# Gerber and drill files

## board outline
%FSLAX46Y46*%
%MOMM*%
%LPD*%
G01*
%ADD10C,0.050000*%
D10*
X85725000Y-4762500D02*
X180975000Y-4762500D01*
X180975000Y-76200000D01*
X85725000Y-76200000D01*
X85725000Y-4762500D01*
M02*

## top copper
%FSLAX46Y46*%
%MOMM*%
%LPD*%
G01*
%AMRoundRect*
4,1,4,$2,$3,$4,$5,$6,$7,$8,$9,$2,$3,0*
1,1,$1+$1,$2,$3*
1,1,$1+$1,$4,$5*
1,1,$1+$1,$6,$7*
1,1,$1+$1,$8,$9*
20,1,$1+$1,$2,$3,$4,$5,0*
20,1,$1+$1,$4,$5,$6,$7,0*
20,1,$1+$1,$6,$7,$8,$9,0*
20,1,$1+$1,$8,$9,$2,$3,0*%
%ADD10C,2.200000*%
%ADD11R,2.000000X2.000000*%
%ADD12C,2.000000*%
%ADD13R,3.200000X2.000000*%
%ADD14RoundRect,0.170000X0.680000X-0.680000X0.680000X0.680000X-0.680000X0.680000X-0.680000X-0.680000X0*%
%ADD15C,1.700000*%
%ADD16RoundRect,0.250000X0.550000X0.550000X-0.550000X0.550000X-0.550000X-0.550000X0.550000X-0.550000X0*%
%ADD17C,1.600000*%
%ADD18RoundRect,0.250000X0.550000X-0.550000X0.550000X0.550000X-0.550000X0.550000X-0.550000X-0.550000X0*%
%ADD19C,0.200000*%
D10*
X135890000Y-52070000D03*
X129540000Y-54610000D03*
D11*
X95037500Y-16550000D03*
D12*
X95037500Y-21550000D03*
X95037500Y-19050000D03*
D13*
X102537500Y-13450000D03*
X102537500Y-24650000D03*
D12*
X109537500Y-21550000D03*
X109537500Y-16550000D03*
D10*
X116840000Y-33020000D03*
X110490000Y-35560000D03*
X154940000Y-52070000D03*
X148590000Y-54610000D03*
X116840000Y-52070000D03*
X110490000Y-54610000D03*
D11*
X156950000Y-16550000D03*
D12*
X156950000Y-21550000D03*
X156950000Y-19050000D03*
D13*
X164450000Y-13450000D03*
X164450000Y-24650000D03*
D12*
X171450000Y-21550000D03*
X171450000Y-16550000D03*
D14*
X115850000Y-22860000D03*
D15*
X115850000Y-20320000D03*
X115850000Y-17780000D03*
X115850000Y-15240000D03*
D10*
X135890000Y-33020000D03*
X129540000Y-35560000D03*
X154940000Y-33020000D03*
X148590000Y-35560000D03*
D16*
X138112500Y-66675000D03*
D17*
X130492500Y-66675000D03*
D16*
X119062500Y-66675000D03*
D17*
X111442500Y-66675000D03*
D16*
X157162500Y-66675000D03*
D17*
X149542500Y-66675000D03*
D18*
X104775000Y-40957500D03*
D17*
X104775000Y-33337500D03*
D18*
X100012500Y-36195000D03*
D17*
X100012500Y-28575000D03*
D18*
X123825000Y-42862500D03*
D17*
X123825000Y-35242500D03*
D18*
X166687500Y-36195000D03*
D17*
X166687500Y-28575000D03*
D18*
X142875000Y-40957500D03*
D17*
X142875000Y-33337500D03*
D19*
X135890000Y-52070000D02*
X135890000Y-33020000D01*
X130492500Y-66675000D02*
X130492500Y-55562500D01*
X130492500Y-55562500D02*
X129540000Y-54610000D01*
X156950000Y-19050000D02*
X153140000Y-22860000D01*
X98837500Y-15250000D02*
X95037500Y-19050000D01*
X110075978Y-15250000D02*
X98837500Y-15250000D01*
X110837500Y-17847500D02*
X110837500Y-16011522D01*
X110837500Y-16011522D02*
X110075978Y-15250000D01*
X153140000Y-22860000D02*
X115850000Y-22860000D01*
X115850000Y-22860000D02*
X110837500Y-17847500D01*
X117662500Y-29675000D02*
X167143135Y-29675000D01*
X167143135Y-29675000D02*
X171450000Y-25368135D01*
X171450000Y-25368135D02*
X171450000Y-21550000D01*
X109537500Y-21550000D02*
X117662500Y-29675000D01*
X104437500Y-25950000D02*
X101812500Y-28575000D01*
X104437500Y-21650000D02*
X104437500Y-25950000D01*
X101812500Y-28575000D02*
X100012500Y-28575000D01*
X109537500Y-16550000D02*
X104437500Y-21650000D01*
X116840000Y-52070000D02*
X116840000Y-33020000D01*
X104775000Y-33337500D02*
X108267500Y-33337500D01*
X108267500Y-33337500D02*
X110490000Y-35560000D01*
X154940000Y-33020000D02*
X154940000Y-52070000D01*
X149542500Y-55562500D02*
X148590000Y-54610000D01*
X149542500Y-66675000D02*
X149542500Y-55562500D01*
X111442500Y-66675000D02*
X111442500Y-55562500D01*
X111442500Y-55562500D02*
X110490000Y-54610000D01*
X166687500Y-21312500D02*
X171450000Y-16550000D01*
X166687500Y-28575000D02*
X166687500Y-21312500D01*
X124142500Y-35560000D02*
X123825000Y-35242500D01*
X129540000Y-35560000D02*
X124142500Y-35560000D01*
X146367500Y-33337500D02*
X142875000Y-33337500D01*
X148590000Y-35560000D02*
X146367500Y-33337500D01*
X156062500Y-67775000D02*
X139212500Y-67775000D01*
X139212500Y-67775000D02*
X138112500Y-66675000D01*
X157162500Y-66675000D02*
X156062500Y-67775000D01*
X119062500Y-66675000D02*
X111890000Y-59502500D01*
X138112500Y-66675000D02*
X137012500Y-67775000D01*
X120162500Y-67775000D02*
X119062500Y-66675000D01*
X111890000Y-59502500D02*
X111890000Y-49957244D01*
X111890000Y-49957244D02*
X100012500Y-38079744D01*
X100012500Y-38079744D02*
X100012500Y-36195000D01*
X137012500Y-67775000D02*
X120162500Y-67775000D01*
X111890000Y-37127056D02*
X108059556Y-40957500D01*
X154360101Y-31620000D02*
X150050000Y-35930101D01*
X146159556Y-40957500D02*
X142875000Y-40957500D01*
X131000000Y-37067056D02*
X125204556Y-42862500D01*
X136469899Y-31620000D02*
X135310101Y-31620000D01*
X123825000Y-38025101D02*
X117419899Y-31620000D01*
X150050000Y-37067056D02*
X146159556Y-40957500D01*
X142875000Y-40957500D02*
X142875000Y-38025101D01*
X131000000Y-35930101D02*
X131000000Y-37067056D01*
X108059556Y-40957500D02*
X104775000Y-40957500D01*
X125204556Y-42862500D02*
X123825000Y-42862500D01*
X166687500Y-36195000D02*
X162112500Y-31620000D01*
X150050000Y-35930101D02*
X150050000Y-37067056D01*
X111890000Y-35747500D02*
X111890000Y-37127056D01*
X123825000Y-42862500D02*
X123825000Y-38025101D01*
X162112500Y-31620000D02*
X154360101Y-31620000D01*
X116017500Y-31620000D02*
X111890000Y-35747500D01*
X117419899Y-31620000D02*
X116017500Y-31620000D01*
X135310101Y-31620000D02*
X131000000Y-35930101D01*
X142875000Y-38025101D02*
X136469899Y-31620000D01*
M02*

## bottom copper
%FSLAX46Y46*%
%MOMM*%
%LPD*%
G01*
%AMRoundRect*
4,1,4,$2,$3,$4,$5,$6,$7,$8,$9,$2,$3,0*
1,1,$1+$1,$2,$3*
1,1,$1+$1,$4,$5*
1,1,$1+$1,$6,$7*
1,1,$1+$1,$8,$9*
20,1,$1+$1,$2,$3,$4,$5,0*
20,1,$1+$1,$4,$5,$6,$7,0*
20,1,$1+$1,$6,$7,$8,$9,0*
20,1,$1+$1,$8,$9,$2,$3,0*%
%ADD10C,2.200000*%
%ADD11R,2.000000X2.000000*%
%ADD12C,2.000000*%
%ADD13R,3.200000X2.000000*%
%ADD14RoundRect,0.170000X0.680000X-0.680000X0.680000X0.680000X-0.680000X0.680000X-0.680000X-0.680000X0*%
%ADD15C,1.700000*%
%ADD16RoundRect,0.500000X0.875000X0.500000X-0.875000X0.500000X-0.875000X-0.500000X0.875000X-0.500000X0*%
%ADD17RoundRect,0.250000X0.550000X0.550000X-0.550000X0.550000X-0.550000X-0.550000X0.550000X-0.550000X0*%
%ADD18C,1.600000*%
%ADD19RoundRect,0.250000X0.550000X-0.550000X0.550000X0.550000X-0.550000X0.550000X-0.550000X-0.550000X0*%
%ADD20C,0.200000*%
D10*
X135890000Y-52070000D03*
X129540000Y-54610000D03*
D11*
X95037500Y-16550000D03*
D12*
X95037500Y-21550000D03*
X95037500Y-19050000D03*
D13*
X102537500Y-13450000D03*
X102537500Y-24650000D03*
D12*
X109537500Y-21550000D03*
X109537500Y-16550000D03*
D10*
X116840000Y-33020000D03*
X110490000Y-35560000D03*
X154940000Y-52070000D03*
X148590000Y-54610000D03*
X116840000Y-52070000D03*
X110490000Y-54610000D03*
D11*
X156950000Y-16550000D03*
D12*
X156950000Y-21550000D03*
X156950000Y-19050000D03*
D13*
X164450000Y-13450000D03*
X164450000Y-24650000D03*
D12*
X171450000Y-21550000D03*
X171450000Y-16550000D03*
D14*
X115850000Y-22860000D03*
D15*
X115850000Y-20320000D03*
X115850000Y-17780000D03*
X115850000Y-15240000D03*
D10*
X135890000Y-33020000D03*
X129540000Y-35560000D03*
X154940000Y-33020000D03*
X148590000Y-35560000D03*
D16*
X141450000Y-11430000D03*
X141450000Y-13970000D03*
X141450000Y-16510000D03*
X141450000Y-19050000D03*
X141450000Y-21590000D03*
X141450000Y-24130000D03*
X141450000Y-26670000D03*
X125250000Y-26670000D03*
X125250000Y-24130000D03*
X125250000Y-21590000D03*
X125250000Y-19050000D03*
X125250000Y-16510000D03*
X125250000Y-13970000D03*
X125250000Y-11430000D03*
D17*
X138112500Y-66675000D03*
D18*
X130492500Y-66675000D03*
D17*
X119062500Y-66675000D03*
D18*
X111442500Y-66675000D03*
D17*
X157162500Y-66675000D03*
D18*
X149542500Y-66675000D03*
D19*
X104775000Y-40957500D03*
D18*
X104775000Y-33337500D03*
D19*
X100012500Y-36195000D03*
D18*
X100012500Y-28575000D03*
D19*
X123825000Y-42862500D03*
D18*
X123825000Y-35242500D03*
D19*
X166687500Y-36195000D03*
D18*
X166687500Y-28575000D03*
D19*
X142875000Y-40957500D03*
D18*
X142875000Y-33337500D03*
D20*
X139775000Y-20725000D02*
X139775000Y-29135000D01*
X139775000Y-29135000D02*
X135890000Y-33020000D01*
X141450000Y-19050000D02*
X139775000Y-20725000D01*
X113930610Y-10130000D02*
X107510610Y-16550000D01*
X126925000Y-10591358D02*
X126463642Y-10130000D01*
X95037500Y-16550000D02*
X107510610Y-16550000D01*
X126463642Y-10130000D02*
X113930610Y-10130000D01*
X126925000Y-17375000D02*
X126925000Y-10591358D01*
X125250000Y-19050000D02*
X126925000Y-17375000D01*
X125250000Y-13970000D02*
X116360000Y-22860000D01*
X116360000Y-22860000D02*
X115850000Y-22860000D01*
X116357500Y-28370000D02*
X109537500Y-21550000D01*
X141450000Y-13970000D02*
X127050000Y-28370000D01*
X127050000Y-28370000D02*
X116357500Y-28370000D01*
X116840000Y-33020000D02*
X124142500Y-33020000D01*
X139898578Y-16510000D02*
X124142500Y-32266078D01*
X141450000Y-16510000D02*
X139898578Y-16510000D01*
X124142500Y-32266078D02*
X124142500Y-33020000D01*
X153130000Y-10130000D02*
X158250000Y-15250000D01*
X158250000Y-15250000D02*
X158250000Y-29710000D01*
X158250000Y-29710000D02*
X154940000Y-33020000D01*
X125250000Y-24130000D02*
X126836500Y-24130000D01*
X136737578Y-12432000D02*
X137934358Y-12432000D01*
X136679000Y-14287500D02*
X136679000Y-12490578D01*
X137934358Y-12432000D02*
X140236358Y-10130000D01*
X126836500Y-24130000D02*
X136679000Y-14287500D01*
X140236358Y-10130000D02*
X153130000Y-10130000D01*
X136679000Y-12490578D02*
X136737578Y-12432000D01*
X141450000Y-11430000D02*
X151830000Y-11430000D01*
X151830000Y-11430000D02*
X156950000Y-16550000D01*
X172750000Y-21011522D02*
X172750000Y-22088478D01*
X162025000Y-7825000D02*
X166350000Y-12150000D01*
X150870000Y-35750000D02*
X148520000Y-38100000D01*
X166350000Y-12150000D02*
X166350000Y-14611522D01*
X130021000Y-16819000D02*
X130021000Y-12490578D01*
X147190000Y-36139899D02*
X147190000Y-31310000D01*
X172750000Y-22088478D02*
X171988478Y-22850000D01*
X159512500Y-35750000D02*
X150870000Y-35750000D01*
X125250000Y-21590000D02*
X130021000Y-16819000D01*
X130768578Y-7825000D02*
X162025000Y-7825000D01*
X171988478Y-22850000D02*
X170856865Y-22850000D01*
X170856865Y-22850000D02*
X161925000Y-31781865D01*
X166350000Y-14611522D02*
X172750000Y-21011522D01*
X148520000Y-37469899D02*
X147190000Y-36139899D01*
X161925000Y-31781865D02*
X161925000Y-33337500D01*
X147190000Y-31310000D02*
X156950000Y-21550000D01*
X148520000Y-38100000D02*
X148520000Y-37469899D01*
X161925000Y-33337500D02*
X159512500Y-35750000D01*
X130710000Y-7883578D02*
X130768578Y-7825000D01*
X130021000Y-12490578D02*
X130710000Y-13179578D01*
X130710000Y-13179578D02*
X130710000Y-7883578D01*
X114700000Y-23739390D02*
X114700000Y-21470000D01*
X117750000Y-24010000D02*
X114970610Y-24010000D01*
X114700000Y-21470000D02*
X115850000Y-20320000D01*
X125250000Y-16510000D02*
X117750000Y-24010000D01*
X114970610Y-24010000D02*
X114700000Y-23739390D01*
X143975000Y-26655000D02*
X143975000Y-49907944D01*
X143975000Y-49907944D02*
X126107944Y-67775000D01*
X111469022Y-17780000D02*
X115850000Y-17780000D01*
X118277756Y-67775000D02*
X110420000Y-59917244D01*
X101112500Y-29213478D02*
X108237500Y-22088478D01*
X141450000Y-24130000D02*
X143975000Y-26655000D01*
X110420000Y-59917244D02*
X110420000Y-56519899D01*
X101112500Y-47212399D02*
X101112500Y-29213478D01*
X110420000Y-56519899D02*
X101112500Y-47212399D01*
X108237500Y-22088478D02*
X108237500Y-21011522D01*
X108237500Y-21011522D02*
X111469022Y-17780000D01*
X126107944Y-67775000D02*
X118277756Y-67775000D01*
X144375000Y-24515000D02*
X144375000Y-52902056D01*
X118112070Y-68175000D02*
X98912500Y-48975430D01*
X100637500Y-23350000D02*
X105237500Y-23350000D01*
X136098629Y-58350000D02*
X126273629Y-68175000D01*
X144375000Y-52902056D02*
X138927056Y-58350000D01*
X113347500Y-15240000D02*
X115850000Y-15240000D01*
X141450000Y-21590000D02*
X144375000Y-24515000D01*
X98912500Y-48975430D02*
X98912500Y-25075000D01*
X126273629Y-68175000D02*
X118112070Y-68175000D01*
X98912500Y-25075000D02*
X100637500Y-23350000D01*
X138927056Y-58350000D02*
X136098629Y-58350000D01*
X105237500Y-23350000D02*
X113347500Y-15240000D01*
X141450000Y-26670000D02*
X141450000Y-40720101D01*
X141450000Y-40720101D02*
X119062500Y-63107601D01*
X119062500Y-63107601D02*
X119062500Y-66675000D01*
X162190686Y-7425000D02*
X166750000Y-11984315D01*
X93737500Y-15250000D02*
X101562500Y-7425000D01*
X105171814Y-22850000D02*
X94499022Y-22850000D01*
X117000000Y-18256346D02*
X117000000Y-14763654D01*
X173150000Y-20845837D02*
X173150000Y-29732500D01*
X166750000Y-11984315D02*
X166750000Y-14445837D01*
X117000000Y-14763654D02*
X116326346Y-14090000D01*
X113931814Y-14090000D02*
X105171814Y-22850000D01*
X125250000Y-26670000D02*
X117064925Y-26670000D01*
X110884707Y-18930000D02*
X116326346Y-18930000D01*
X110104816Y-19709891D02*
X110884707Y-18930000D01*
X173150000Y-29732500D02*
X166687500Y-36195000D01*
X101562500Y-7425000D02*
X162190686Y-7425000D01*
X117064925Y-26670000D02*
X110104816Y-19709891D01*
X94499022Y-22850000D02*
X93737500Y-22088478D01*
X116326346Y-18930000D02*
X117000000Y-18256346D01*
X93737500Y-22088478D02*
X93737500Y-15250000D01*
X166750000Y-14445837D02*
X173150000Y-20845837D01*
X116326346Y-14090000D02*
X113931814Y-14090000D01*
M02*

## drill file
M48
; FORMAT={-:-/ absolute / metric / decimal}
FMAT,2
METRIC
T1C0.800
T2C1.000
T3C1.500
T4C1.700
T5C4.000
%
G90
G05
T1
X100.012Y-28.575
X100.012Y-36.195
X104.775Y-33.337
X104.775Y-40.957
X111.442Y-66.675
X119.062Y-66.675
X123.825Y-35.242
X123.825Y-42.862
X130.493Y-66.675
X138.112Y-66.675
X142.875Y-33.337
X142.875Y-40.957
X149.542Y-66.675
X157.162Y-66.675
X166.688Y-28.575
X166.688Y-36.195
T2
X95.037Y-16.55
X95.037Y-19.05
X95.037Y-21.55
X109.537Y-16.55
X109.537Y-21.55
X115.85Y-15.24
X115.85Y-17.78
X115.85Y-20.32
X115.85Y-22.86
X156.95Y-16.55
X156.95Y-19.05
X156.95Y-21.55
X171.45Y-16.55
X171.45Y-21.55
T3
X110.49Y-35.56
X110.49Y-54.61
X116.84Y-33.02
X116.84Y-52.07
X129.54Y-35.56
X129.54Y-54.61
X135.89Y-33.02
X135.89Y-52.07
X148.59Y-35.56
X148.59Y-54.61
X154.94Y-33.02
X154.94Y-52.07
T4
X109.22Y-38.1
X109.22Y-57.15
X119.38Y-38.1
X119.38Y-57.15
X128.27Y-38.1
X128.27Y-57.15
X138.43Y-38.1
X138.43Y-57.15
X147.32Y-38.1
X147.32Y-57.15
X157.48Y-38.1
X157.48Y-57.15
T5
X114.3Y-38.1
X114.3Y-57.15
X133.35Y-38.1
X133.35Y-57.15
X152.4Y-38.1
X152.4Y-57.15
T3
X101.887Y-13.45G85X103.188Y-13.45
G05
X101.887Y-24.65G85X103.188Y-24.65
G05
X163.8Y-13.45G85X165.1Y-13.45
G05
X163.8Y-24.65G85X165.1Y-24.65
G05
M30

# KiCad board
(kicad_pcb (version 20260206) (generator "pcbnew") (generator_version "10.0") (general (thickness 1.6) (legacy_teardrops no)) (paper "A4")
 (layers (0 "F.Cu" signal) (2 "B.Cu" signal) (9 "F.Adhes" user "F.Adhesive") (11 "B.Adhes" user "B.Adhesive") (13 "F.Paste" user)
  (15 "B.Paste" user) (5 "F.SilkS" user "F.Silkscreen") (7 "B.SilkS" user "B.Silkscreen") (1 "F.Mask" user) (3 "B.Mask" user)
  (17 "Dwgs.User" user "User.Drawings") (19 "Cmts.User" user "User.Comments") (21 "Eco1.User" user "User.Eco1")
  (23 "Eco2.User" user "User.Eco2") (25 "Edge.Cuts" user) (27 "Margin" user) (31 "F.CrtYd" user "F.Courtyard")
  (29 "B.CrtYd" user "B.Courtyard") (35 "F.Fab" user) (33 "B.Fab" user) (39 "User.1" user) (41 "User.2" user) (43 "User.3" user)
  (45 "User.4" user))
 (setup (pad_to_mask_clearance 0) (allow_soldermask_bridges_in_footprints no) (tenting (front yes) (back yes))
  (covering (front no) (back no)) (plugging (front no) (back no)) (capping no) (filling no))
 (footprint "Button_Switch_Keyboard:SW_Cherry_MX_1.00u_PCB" (layer "F.Cu") (at 135.89 52.07)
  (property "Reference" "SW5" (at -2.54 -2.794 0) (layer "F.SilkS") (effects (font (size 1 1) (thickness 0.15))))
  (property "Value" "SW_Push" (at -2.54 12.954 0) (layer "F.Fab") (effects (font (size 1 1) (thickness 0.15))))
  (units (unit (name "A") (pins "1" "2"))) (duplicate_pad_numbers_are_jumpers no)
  (pad "" np_thru_hole circle (at -7.62 5.08) (size 1.7 1.7) (drill 1.7) (layers "*.Cu" "*.Mask"))
  (pad "" np_thru_hole circle (at -2.54 5.08) (size 4 4) (drill 4) (layers "*.Cu" "*.Mask"))
  (pad "" np_thru_hole circle (at 2.54 5.08) (size 1.7 1.7) (drill 1.7) (layers "*.Cu" "*.Mask"))
  (pad "1" thru_hole circle (at 0 0) (size 2.2 2.2) (drill 1.5) (layers "*.Cu" "*.Mask") (remove_unused_layers no) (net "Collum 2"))
  (pad "2" thru_hole circle (at -6.35 2.54) (size 2.2 2.2) (drill 1.5) (layers "*.Cu" "*.Mask") (remove_unused_layers no) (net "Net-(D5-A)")))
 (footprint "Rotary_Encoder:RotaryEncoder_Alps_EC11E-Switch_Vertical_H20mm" (layer "F.Cu") (at 95.0375 16.55)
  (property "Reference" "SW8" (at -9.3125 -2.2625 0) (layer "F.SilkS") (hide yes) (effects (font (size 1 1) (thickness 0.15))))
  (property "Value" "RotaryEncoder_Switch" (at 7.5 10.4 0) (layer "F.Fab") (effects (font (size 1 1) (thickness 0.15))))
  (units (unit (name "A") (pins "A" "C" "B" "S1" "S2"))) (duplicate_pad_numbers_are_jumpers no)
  (pad "A" thru_hole rect (at 0 0) (size 2 2) (drill 1) (layers "*.Cu" "*.Mask") (remove_unused_layers no) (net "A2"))
  (pad "B" thru_hole circle (at 0 5) (size 2 2) (drill 1) (layers "*.Cu" "*.Mask") (remove_unused_layers no) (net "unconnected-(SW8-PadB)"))
  (pad "C" thru_hole circle (at 0 2.5) (size 2 2) (drill 1) (layers "*.Cu" "*.Mask") (remove_unused_layers no) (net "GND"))
  (pad "MP" thru_hole rect (at 7.5 -3.1) (size 3.2 2) (drill oval 2.8 1.5) (layers "*.Cu" "*.Mask") (remove_unused_layers no))
  (pad "MP" thru_hole rect (at 7.5 8.1) (size 3.2 2) (drill oval 2.8 1.5) (layers "*.Cu" "*.Mask") (remove_unused_layers no))
  (pad "S1" thru_hole circle (at 14.5 5) (size 2 2) (drill 1) (layers "*.Cu" "*.Mask") (remove_unused_layers no) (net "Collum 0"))
  (pad "S2" thru_hole circle (at 14.5 0) (size 2 2) (drill 1) (layers "*.Cu" "*.Mask") (remove_unused_layers no) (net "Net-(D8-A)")))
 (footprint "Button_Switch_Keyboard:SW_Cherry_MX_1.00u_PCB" (layer "F.Cu") (at 116.84 33.02)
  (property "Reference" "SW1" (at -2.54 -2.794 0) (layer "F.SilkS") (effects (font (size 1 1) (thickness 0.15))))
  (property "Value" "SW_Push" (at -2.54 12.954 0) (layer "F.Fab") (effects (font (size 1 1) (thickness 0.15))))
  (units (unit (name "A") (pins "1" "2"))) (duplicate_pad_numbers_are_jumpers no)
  (pad "" np_thru_hole circle (at -7.62 5.08) (size 1.7 1.7) (drill 1.7) (layers "*.Cu" "*.Mask"))
  (pad "" np_thru_hole circle (at -2.54 5.08) (size 4 4) (drill 4) (layers "*.Cu" "*.Mask"))
  (pad "" np_thru_hole circle (at 2.54 5.08) (size 1.7 1.7) (drill 1.7) (layers "*.Cu" "*.Mask"))
  (pad "1" thru_hole circle (at 0 0) (size 2.2 2.2) (drill 1.5) (layers "*.Cu" "*.Mask") (remove_unused_layers no) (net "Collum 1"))
  (pad "2" thru_hole circle (at -6.35 2.54) (size 2.2 2.2) (drill 1.5) (layers "*.Cu" "*.Mask") (remove_unused_layers no) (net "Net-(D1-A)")))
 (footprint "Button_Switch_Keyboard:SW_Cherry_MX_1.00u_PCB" (layer "F.Cu") (at 154.94 52.07)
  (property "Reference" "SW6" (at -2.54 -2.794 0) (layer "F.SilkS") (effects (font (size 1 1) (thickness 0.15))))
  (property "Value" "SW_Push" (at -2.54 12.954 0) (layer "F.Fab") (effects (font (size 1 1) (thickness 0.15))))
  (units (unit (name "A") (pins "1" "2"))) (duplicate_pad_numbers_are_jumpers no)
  (pad "" np_thru_hole circle (at -7.62 5.08) (size 1.7 1.7) (drill 1.7) (layers "*.Cu" "*.Mask"))
  (pad "" np_thru_hole circle (at -2.54 5.08) (size 4 4) (drill 4) (layers "*.Cu" "*.Mask"))
  (pad "" np_thru_hole circle (at 2.54 5.08) (size 1.7 1.7) (drill 1.7) (layers "*.Cu" "*.Mask"))
  (pad "1" thru_hole circle (at 0 0) (size 2.2 2.2) (drill 1.5) (layers "*.Cu" "*.Mask") (remove_unused_layers no) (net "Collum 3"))
  (pad "2" thru_hole circle (at -6.35 2.54) (size 2.2 2.2) (drill 1.5) (layers "*.Cu" "*.Mask") (remove_unused_layers no) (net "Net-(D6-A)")))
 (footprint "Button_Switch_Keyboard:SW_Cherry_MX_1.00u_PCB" (layer "F.Cu") (at 116.84 52.07)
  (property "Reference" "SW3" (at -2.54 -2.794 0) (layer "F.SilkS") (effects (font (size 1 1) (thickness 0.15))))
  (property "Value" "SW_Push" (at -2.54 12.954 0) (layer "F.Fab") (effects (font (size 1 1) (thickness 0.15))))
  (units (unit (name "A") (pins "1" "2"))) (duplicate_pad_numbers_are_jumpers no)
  (pad "" np_thru_hole circle (at -7.62 5.08) (size 1.7 1.7) (drill 1.7) (layers "*.Cu" "*.Mask"))
  (pad "" np_thru_hole circle (at -2.54 5.08) (size 4 4) (drill 4) (layers "*.Cu" "*.Mask"))
  (pad "" np_thru_hole circle (at 2.54 5.08) (size 1.7 1.7) (drill 1.7) (layers "*.Cu" "*.Mask"))
  (pad "1" thru_hole circle (at 0 0) (size 2.2 2.2) (drill 1.5) (layers "*.Cu" "*.Mask") (remove_unused_layers no) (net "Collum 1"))
  (pad "2" thru_hole circle (at -6.35 2.54) (size 2.2 2.2) (drill 1.5) (layers "*.Cu" "*.Mask") (remove_unused_layers no) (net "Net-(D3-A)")))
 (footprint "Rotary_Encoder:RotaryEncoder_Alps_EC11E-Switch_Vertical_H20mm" (layer "F.Cu") (at 156.95 16.55)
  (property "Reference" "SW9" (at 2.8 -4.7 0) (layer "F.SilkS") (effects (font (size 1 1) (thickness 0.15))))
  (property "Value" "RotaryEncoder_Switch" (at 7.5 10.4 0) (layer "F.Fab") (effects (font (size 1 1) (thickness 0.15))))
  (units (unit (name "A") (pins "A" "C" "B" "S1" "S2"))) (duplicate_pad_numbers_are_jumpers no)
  (pad "A" thru_hole rect (at 0 0) (size 2 2) (drill 1) (layers "*.Cu" "*.Mask") (remove_unused_layers no) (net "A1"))
  (pad "B" thru_hole circle (at 0 5) (size 2 2) (drill 1) (layers "*.Cu" "*.Mask") (remove_unused_layers no) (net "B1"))
  (pad "C" thru_hole circle (at 0 2.5) (size 2 2) (drill 1) (layers "*.Cu" "*.Mask") (remove_unused_layers no) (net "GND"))
  (pad "MP" thru_hole rect (at 7.5 -3.1) (size 3.2 2) (drill oval 2.8 1.5) (layers "*.Cu" "*.Mask") (remove_unused_layers no))
  (pad "MP" thru_hole rect (at 7.5 8.1) (size 3.2 2) (drill oval 2.8 1.5) (layers "*.Cu" "*.Mask") (remove_unused_layers no))
  (pad "S1" thru_hole circle (at 14.5 5) (size 2 2) (drill 1) (layers "*.Cu" "*.Mask") (remove_unused_layers no) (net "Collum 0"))
  (pad "S2" thru_hole circle (at 14.5 0) (size 2 2) (drill 1) (layers "*.Cu" "*.Mask") (remove_unused_layers no) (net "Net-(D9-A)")))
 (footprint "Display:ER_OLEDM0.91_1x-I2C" (layer "F.Cu") (at 115.85 22.86 90)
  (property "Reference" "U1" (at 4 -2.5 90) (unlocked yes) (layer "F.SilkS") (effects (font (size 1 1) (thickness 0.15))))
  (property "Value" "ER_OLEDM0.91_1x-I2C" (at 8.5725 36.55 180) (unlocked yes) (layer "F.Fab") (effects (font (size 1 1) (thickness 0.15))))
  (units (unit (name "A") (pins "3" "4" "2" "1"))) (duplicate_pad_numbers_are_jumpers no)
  (pad "1" thru_hole roundrect (at 0 0 90) (size 1.7 1.7) (drill 1) (layers "*.Cu" "*.Mask") (remove_unused_layers no)
   (roundrect_rratio 0.1) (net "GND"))
  (pad "2" thru_hole circle (at 2.54 0 90) (size 1.7 1.7) (drill 1) (layers "*.Cu" "*.Mask") (remove_unused_layers no) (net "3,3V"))
  (pad "3" thru_hole circle (at 5.08 0 90) (size 1.7 1.7) (drill 1) (layers "*.Cu" "*.Mask") (remove_unused_layers no) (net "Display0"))
  (pad "4" thru_hole circle (at 7.62 0 90) (size 1.7 1.7) (drill 1) (layers "*.Cu" "*.Mask") (remove_unused_layers no) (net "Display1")))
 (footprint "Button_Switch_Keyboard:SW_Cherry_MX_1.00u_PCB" (layer "F.Cu") (at 135.89 33.02)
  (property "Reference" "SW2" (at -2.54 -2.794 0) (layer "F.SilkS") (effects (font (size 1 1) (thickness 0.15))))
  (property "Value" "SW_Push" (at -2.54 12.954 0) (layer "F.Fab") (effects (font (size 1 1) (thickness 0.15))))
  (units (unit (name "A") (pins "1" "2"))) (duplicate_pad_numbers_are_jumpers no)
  (pad "" np_thru_hole circle (at -7.62 5.08) (size 1.7 1.7) (drill 1.7) (layers "*.Cu" "*.Mask"))
  (pad "" np_thru_hole circle (at -2.54 5.08) (size 4 4) (drill 4) (layers "*.Cu" "*.Mask"))
  (pad "" np_thru_hole circle (at 2.54 5.08) (size 1.7 1.7) (drill 1.7) (layers "*.Cu" "*.Mask"))
  (pad "1" thru_hole circle (at 0 0) (size 2.2 2.2) (drill 1.5) (layers "*.Cu" "*.Mask") (remove_unused_layers no) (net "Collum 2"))
  (pad "2" thru_hole circle (at -6.35 2.54) (size 2.2 2.2) (drill 1.5) (layers "*.Cu" "*.Mask") (remove_unused_layers no) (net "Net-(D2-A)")))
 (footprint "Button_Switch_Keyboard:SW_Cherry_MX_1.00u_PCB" (layer "F.Cu") (at 154.94 33.02)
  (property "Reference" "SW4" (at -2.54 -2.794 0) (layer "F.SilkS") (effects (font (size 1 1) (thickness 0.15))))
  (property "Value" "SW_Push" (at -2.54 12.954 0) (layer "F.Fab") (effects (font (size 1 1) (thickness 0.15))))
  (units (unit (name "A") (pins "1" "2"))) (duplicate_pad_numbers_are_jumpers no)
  (pad "" np_thru_hole circle (at -7.62 5.08) (size 1.7 1.7) (drill 1.7) (layers "*.Cu" "*.Mask"))
  (pad "" np_thru_hole circle (at -2.54 5.08) (size 4 4) (drill 4) (layers "*.Cu" "*.Mask"))
  (pad "" np_thru_hole circle (at 2.54 5.08) (size 1.7 1.7) (drill 1.7) (layers "*.Cu" "*.Mask"))
  (pad "1" thru_hole circle (at 0 0) (size 2.2 2.2) (drill 1.5) (layers "*.Cu" "*.Mask") (remove_unused_layers no) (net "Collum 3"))
  (pad "2" thru_hole circle (at -6.35 2.54) (size 2.2 2.2) (drill 1.5) (layers "*.Cu" "*.Mask") (remove_unused_layers no) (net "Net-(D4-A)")))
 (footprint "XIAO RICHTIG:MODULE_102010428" (layer "B.Cu") (at 133.35 19.05 180)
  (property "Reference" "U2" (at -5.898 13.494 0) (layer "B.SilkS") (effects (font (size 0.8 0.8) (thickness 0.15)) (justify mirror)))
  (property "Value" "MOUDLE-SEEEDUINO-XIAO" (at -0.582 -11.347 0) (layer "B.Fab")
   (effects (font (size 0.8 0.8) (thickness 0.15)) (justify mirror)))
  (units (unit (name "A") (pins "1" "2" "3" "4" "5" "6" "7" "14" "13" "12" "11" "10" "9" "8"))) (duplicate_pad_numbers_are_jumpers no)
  (pad "1" smd roundrect (at -8.1 7.62 180) (size 2.75 2) (layers "B.Cu" "B.Mask" "B.Paste") (roundrect_rratio 0.25) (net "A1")
   (solder_mask_margin 0.102))
  (pad "2" smd roundrect (at -8.1 5.08 180) (size 2.75 2) (layers "B.Cu" "B.Mask" "B.Paste") (roundrect_rratio 0.25) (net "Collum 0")
   (solder_mask_margin 0.102))
  (pad "3" smd roundrect (at -8.1 2.54 180) (size 2.75 2) (layers "B.Cu" "B.Mask" "B.Paste") (roundrect_rratio 0.25) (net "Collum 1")
   (solder_mask_margin 0.102))
  (pad "4" smd roundrect (at -8.1 0 180) (size 2.75 2) (layers "B.Cu" "B.Mask" "B.Paste") (roundrect_rratio 0.25) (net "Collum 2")
   (solder_mask_margin 0.102))
  (pad "5" smd roundrect (at -8.1 -2.54 180) (size 2.75 2) (layers "B.Cu" "B.Mask" "B.Paste") (roundrect_rratio 0.25) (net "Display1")
   (solder_mask_margin 0.102))
  (pad "6" smd roundrect (at -8.1 -5.08 180) (size 2.75 2) (layers "B.Cu" "B.Mask" "B.Paste") (roundrect_rratio 0.25) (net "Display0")
   (solder_mask_margin 0.102))
  (pad "7" smd roundrect (at -8.1 -7.62 180) (size 2.75 2) (layers "B.Cu" "B.Mask" "B.Paste") (roundrect_rratio 0.25) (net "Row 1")
   (solder_mask_margin 0.102))
  (pad "8" smd roundrect (at 8.1 -7.62 180) (size 2.75 2) (layers "B.Cu" "B.Mask" "B.Paste") (roundrect_rratio 0.25) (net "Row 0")
   (solder_mask_margin 0.102))
  (pad "9" smd roundrect (at 8.1 -5.08 180) (size 2.75 2) (layers "B.Cu" "B.Mask" "B.Paste") (roundrect_rratio 0.25) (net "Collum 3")
   (solder_mask_margin 0.102))
  (pad "10" smd roundrect (at 8.1 -2.54 180) (size 2.75 2) (layers "B.Cu" "B.Mask" "B.Paste") (roundrect_rratio 0.25) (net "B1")
   (solder_mask_margin 0.102))
  (pad "11" smd roundrect (at 8.1 0 180) (size 2.75 2) (layers "B.Cu" "B.Mask" "B.Paste") (roundrect_rratio 0.25) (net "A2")
   (solder_mask_margin 0.102))
  (pad "12" smd roundrect (at 8.1 2.54 180) (size 2.75 2) (layers "B.Cu" "B.Mask" "B.Paste") (roundrect_rratio 0.25) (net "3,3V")
   (solder_mask_margin 0.102))
  (pad "13" smd roundrect (at 8.1 5.08 180) (size 2.75 2) (layers "B.Cu" "B.Mask" "B.Paste") (roundrect_rratio 0.25) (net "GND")
   (solder_mask_margin 0.102))
  (pad "14" smd roundrect (at 8.1 7.62 180) (size 2.75 2) (layers "B.Cu" "B.Mask" "B.Paste") (roundrect_rratio 0.25)
   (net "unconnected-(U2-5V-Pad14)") (solder_mask_margin 0.102))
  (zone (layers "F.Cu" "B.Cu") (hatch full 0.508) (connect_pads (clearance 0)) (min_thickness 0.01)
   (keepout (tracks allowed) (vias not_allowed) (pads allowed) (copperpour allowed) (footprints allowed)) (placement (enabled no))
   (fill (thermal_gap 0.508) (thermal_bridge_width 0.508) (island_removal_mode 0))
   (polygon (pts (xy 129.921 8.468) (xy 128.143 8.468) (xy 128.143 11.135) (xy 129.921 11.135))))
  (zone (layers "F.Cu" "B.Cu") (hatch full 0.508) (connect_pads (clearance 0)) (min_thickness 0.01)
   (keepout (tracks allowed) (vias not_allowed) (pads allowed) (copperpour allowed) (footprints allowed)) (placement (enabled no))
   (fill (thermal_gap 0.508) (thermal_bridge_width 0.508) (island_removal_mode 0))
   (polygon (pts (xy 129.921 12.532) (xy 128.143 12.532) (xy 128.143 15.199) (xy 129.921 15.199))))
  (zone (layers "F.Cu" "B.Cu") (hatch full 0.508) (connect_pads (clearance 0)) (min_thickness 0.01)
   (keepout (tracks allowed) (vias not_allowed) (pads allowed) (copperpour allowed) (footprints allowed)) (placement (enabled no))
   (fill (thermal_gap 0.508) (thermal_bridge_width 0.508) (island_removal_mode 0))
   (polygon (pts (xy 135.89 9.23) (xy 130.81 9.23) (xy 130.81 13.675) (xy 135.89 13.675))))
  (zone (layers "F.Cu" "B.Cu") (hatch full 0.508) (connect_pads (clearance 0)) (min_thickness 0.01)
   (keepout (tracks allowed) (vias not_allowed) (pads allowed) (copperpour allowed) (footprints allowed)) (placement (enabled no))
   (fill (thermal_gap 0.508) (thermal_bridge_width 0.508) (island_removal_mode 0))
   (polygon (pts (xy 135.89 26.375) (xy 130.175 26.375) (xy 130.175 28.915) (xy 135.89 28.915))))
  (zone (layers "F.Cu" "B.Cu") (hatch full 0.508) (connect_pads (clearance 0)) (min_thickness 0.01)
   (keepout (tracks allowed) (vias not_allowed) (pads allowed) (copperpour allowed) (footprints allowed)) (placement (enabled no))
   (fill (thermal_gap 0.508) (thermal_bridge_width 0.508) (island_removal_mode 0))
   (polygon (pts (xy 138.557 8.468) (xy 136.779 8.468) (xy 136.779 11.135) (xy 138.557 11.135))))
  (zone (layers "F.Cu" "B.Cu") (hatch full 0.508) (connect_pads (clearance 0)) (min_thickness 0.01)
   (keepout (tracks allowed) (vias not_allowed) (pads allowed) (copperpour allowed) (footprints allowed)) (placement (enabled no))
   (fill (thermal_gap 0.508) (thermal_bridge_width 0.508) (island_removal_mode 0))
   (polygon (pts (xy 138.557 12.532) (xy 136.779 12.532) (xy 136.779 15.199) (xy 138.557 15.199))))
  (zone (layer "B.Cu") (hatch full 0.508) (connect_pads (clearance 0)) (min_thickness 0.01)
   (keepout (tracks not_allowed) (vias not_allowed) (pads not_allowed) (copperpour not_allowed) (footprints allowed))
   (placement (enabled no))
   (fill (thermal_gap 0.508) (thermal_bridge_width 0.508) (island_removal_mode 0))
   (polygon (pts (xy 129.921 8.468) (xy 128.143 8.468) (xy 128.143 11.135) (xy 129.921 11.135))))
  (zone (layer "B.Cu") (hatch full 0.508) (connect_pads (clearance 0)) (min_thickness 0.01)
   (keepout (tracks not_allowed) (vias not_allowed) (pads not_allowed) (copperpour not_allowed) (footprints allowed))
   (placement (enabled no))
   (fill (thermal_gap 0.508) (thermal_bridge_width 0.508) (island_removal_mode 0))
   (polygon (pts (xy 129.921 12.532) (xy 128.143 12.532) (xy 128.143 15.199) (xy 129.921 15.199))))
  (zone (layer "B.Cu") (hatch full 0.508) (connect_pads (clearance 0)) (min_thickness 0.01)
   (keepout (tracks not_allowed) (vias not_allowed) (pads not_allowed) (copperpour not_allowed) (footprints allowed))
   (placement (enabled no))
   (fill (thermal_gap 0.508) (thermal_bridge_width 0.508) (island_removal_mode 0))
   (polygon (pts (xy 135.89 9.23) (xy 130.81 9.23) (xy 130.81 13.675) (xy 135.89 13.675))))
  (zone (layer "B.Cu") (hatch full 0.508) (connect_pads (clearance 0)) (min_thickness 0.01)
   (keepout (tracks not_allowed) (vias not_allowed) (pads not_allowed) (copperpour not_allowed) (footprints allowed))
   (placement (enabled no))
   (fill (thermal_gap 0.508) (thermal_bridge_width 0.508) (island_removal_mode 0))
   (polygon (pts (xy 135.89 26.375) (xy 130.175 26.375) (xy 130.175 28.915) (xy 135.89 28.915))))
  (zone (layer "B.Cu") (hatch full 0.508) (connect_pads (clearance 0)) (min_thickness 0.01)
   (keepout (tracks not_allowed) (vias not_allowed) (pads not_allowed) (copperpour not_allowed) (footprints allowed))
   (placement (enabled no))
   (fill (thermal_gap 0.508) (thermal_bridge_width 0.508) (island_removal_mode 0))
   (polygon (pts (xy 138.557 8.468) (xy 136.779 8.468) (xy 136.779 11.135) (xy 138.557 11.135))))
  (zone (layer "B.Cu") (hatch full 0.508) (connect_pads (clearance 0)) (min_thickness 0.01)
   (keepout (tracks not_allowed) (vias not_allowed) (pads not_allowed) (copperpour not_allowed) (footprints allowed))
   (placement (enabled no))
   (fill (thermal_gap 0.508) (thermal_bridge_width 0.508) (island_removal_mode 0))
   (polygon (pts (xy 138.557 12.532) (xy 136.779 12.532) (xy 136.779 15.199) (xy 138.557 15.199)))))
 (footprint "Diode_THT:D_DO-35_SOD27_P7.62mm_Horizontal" (layer "B.Cu") (at 138.1125 66.675 180)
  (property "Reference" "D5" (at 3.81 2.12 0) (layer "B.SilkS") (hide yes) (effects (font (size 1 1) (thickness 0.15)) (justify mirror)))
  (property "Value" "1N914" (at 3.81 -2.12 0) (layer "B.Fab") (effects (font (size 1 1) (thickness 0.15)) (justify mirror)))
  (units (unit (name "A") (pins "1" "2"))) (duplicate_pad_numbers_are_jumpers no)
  (pad "1" thru_hole roundrect (at 0 0 180) (size 1.6 1.6) (drill 0.8) (layers "*.Cu" "*.Mask") (remove_unused_layers no)
   (roundrect_rratio 0.15625) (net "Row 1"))
  (pad "2" thru_hole circle (at 7.62 0 180) (size 1.6 1.6) (drill 0.8) (layers "*.Cu" "*.Mask") (remove_unused_layers no) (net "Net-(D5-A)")))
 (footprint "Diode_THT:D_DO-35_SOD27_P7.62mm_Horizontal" (layer "B.Cu") (at 119.0625 66.675 180)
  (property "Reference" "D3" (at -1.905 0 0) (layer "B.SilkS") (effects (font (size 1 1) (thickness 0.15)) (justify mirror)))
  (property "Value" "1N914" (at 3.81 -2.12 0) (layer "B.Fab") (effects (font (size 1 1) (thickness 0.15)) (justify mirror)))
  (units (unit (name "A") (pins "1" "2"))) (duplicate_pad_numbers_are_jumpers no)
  (pad "1" thru_hole roundrect (at 0 0 180) (size 1.6 1.6) (drill 0.8) (layers "*.Cu" "*.Mask") (remove_unused_layers no)
   (roundrect_rratio 0.15625) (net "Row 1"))
  (pad "2" thru_hole circle (at 7.62 0 180) (size 1.6 1.6) (drill 0.8) (layers "*.Cu" "*.Mask") (remove_unused_layers no) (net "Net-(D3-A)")))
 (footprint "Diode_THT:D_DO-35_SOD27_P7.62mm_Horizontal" (layer "B.Cu") (at 157.1625 66.675 180)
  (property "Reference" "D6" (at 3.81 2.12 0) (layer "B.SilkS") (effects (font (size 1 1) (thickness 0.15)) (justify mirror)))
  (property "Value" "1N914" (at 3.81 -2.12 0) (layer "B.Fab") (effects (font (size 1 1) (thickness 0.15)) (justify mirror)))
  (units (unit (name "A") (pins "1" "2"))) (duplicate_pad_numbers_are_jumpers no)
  (pad "1" thru_hole roundrect (at 0 0 180) (size 1.6 1.6) (drill 0.8) (layers "*.Cu" "*.Mask") (remove_unused_layers no)
   (roundrect_rratio 0.15625) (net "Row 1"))
  (pad "2" thru_hole circle (at 7.62 0 180) (size 1.6 1.6) (drill 0.8) (layers "*.Cu" "*.Mask") (remove_unused_layers no) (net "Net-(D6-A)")))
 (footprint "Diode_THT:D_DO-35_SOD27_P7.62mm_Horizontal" (layer "B.Cu") (at 104.775 40.9575 90)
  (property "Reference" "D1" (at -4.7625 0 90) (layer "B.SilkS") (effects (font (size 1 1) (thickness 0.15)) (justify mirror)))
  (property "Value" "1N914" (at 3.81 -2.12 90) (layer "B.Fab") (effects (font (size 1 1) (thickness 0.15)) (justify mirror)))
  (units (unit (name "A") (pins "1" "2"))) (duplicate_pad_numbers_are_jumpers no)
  (pad "1" thru_hole roundrect (at 0 0 90) (size 1.6 1.6) (drill 0.8) (layers "*.Cu" "*.Mask") (remove_unused_layers no)
   (roundrect_rratio 0.15625) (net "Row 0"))
  (pad "2" thru_hole circle (at 7.62 0 90) (size 1.6 1.6) (drill 0.8) (layers "*.Cu" "*.Mask") (remove_unused_layers no) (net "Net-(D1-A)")))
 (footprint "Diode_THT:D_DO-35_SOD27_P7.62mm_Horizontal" (layer "B.Cu") (at 100.0125 36.195 90)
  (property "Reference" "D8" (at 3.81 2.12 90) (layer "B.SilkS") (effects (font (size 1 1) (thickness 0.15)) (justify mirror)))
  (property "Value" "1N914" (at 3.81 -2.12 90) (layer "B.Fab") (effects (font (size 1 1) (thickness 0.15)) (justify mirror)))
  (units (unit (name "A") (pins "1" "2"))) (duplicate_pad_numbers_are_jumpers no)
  (pad "1" thru_hole roundrect (at 0 0 90) (size 1.6 1.6) (drill 0.8) (layers "*.Cu" "*.Mask") (remove_unused_layers no)
   (roundrect_rratio 0.15625) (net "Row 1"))
  (pad "2" thru_hole circle (at 7.62 0 90) (size 1.6 1.6) (drill 0.8) (layers "*.Cu" "*.Mask") (remove_unused_layers no) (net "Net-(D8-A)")))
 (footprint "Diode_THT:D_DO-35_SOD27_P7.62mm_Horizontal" (layer "B.Cu") (at 123.825 42.8625 90)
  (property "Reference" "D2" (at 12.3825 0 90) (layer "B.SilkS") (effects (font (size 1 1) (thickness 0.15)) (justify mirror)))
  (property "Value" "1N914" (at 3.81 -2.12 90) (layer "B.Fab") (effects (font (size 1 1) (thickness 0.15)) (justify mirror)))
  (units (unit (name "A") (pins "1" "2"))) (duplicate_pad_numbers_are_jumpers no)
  (pad "1" thru_hole roundrect (at 0 0 90) (size 1.6 1.6) (drill 0.8) (layers "*.Cu" "*.Mask") (remove_unused_layers no)
   (roundrect_rratio 0.15625) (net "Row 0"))
  (pad "2" thru_hole circle (at 7.62 0 90) (size 1.6 1.6) (drill 0.8) (layers "*.Cu" "*.Mask") (remove_unused_layers no) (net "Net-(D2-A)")))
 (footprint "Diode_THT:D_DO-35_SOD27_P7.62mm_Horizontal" (layer "B.Cu") (at 166.6875 36.195 90)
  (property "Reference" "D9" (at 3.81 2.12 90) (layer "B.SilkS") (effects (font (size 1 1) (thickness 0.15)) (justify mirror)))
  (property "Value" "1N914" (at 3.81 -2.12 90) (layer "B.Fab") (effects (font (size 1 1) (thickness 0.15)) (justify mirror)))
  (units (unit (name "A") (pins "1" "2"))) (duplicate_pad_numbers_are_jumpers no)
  (pad "1" thru_hole roundrect (at 0 0 90) (size 1.6 1.6) (drill 0.8) (layers "*.Cu" "*.Mask") (remove_unused_layers no)
   (roundrect_rratio 0.15625) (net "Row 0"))
  (pad "2" thru_hole circle (at 7.62 0 90) (size 1.6 1.6) (drill 0.8) (layers "*.Cu" "*.Mask") (remove_unused_layers no) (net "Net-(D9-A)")))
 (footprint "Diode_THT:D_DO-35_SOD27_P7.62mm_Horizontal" (layer "B.Cu") (at 142.875 40.9575 90)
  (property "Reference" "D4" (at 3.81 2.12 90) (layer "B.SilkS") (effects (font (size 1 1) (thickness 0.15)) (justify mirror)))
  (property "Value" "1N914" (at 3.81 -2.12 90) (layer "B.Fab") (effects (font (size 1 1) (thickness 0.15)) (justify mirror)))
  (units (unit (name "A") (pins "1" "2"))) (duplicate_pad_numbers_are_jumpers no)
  (pad "1" thru_hole roundrect (at 0 0 90) (size 1.6 1.6) (drill 0.8) (layers "*.Cu" "*.Mask") (remove_unused_layers no)
   (roundrect_rratio 0.15625) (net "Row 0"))
  (pad "2" thru_hole circle (at 7.62 0 90) (size 1.6 1.6) (drill 0.8) (layers "*.Cu" "*.Mask") (remove_unused_layers no) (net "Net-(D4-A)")))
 (gr_rect (start 85.725 4.7625) (end 180.975 76.2) (stroke (width 0.05) (type default)) (fill no) (layer "Edge.Cuts"))
 (segment (start 135.89 52.07) (end 135.89 33.02) (width 0.2) (layer "F.Cu") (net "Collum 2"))
 (segment (start 139.775 20.725) (end 139.775 29.135) (width 0.2) (layer "B.Cu") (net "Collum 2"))
 (segment (start 139.775 29.135) (end 135.89 33.02) (width 0.2) (layer "B.Cu") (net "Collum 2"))
 (segment (start 141.45 19.05) (end 139.775 20.725) (width 0.2) (layer "B.Cu") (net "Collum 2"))
 (segment (start 130.4925 66.675) (end 130.4925 55.5625) (width 0.2) (layer "F.Cu") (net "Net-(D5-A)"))
 (segment (start 130.4925 55.5625) (end 129.54 54.61) (width 0.2) (layer "F.Cu") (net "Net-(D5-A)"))
 (segment (start 113.93061 10.13) (end 107.51061 16.55) (width 0.2) (layer "B.Cu") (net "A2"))
 (segment (start 126.925 10.591358) (end 126.463642 10.13) (width 0.2) (layer "B.Cu") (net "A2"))
 (segment (start 95.0375 16.55) (end 107.51061 16.55) (width 0.2) (layer "B.Cu") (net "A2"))
 (segment (start 126.463642 10.13) (end 113.93061 10.13) (width 0.2) (layer "B.Cu") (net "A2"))
 (segment (start 126.925 17.375) (end 126.925 10.591358) (width 0.2) (layer "B.Cu") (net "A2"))
 (segment (start 125.25 19.05) (end 126.925 17.375) (width 0.2) (layer "B.Cu") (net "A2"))
 (segment (start 156.95 19.05) (end 153.14 22.86) (width 0.2) (layer "F.Cu") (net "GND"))
 (segment (start 98.8375 15.25) (end 95.0375 19.05) (width 0.2) (layer "F.Cu") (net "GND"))
 (segment (start 110.075978 15.25) (end 98.8375 15.25) (width 0.2) (layer "F.Cu") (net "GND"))
 (segment (start 110.8375 17.8475) (end 110.8375 16.011522) (width 0.2) (layer "F.Cu") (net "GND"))
 (segment (start 110.8375 16.011522) (end 110.075978 15.25) (width 0.2) (layer "F.Cu") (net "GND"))
 (segment (start 153.14 22.86) (end 115.85 22.86) (width 0.2) (layer "F.Cu") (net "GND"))
 (segment (start 115.85 22.86) (end 110.8375 17.8475) (width 0.2) (layer "F.Cu") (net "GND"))
 (segment (start 125.25 13.97) (end 116.36 22.86) (width 0.2) (layer "B.Cu") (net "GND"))
 (segment (start 116.36 22.86) (end 115.85 22.86) (width 0.2) (layer "B.Cu") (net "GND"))
 (segment (start 117.6625 29.675) (end 167.143135 29.675) (width 0.2) (layer "F.Cu") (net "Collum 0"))
 (segment (start 167.143135 29.675) (end 171.45 25.368135) (width 0.2) (layer "F.Cu") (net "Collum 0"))
 (segment (start 171.45 25.368135) (end 171.45 21.55) (width 0.2) (layer "F.Cu") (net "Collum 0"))
 (segment (start 109.5375 21.55) (end 117.6625 29.675) (width 0.2) (layer "F.Cu") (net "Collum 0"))
 (segment (start 116.3575 28.37) (end 109.5375 21.55) (width 0.2) (layer "B.Cu") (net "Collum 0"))
 (segment (start 141.45 13.97) (end 127.05 28.37) (width 0.2) (layer "B.Cu") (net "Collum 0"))
 (segment (start 127.05 28.37) (end 116.3575 28.37) (width 0.2) (layer "B.Cu") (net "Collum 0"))
 (segment (start 104.4375 25.95) (end 101.8125 28.575) (width 0.2) (layer "F.Cu") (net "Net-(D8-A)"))
 (segment (start 104.4375 21.65) (end 104.4375 25.95) (width 0.2) (layer "F.Cu") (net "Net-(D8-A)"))
 (segment (start 101.8125 28.575) (end 100.0125 28.575) (width 0.2) (layer "F.Cu") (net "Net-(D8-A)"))
 (segment (start 109.5375 16.55) (end 104.4375 21.65) (width 0.2) (layer "F.Cu") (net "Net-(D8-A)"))
 (segment (start 116.84 52.07) (end 116.84 33.02) (width 0.2) (layer "F.Cu") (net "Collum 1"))
 (segment (start 116.84 33.02) (end 124.1425 33.02) (width 0.2) (layer "B.Cu") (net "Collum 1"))
 (segment (start 139.898578 16.51) (end 124.1425 32.266078) (width 0.2) (layer "B.Cu") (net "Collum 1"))
 (segment (start 141.45 16.51) (end 139.898578 16.51) (width 0.2) (layer "B.Cu") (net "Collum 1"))
 (segment (start 124.1425 32.266078) (end 124.1425 33.02) (width 0.2) (layer "B.Cu") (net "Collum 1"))
 (segment (start 104.775 33.3375) (end 108.2675 33.3375) (width 0.2) (layer "F.Cu") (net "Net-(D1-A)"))
 (segment (start 108.2675 33.3375) (end 110.49 35.56) (width 0.2) (layer "F.Cu") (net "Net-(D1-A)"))
 (segment (start 154.94 33.02) (end 154.94 52.07) (width 0.2) (layer "F.Cu") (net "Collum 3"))
 (segment (start 153.13 10.13) (end 158.25 15.25) (width 0.2) (layer "B.Cu") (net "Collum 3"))
 (segment (start 158.25 15.25) (end 158.25 29.71) (width 0.2) (layer "B.Cu") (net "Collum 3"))
 (segment (start 158.25 29.71) (end 154.94 33.02) (width 0.2) (layer "B.Cu") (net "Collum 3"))
 (segment (start 125.25 24.13) (end 126.8365 24.13) (width 0.2) (layer "B.Cu") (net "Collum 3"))
 (segment (start 136.737578 12.432) (end 137.934358 12.432) (width 0.2) (layer "B.Cu") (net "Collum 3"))
 (segment (start 136.679 14.2875) (end 136.679 12.490578) (width 0.2) (layer "B.Cu") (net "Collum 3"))
 (segment (start 137.934358 12.432) (end 140.236358 10.13) (width 0.2) (layer "B.Cu") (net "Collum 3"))
 (segment (start 126.8365 24.13) (end 136.679 14.2875) (width 0.2) (layer "B.Cu") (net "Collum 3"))
 (segment (start 140.236358 10.13) (end 153.13 10.13) (width 0.2) (layer "B.Cu") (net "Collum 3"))
 (segment (start 136.679 12.490578) (end 136.737578 12.432) (width 0.2) (layer "B.Cu") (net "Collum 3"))
 (segment (start 149.5425 55.5625) (end 148.59 54.61) (width 0.2) (layer "F.Cu") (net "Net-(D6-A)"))
 (segment (start 149.5425 66.675) (end 149.5425 55.5625) (width 0.2) (layer "F.Cu") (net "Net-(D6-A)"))
 (segment (start 111.4425 66.675) (end 111.4425 55.5625) (width 0.2) (layer "F.Cu") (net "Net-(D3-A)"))
 (segment (start 111.4425 55.5625) (end 110.49 54.61) (width 0.2) (layer "F.Cu") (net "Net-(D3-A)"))
 (segment (start 141.45 11.43) (end 151.83 11.43) (width 0.2) (layer "B.Cu") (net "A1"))
 (segment (start 151.83 11.43) (end 156.95 16.55) (width 0.2) (layer "B.Cu") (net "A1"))
 (segment (start 172.75 21.011522) (end 172.75 22.088478) (width 0.2) (layer "B.Cu") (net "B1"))
 (segment (start 162.025 7.825) (end 166.35 12.15) (width 0.2) (layer "B.Cu") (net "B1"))
 (segment (start 150.87 35.75) (end 148.52 38.1) (width 0.2) (layer "B.Cu") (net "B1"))
 (segment (start 166.35 12.15) (end 166.35 14.611522) (width 0.2) (layer "B.Cu") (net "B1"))
 (segment (start 130.021 16.819) (end 130.021 12.490578) (width 0.2) (layer "B.Cu") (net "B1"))
 (segment (start 147.19 36.139899) (end 147.19 31.31) (width 0.2) (layer "B.Cu") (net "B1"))
 (segment (start 172.75 22.088478) (end 171.988478 22.85) (width 0.2) (layer "B.Cu") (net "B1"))
 (segment (start 159.5125 35.75) (end 150.87 35.75) (width 0.2) (layer "B.Cu") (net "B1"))
 (segment (start 125.25 21.59) (end 130.021 16.819) (width 0.2) (layer "B.Cu") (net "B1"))
 (segment (start 130.768578 7.825) (end 162.025 7.825) (width 0.2) (layer "B.Cu") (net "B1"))
 (segment (start 171.988478 22.85) (end 170.856865 22.85) (width 0.2) (layer "B.Cu") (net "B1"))
 (segment (start 170.856865 22.85) (end 161.925 31.781865) (width 0.2) (layer "B.Cu") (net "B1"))
 (segment (start 166.35 14.611522) (end 172.75 21.011522) (width 0.2) (layer "B.Cu") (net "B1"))
 (segment (start 148.52 37.469899) (end 147.19 36.139899) (width 0.2) (layer "B.Cu") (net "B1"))
 (segment (start 161.925 31.781865) (end 161.925 33.3375) (width 0.2) (layer "B.Cu") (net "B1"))
 (segment (start 147.19 31.31) (end 156.95 21.55) (width 0.2) (layer "B.Cu") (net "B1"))
 (segment (start 148.52 38.1) (end 148.52 37.469899) (width 0.2) (layer "B.Cu") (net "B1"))
 (segment (start 161.925 33.3375) (end 159.5125 35.75) (width 0.2) (layer "B.Cu") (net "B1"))
 (segment (start 130.71 7.883578) (end 130.768578 7.825) (width 0.2) (layer "B.Cu") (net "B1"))
 (segment (start 130.021 12.490578) (end 130.71 13.179578) (width 0.2) (layer "B.Cu") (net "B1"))
 (segment (start 130.71 13.179578) (end 130.71 7.883578) (width 0.2) (layer "B.Cu") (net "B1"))
 (segment (start 166.6875 21.3125) (end 171.45 16.55) (width 0.2) (layer "F.Cu") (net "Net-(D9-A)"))
 (segment (start 166.6875 28.575) (end 166.6875 21.3125) (width 0.2) (layer "F.Cu") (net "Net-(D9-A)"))
 (segment (start 114.7 23.73939) (end 114.7 21.47) (width 0.2) (layer "B.Cu") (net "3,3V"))
 (segment (start 117.75 24.01) (end 114.97061 24.01) (width 0.2) (layer "B.Cu") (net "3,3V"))
 (segment (start 114.7 21.47) (end 115.85 20.32) (width 0.2) (layer "B.Cu") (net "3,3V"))
 (segment (start 125.25 16.51) (end 117.75 24.01) (width 0.2) (layer "B.Cu") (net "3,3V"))
 (segment (start 114.97061 24.01) (end 114.7 23.73939) (width 0.2) (layer "B.Cu") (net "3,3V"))
 (segment (start 143.975 26.655) (end 143.975 49.907944) (width 0.2) (layer "B.Cu") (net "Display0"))
 (segment (start 143.975 49.907944) (end 126.107944 67.775) (width 0.2) (layer "B.Cu") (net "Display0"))
 (segment (start 111.469022 17.78) (end 115.85 17.78) (width 0.2) (layer "B.Cu") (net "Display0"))
 (segment (start 118.277756 67.775) (end 110.42 59.917244) (width 0.2) (layer "B.Cu") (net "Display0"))
 (segment (start 101.1125 29.213478) (end 108.2375 22.088478) (width 0.2) (layer "B.Cu") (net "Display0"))
 (segment (start 141.45 24.13) (end 143.975 26.655) (width 0.2) (layer "B.Cu") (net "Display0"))
 (segment (start 110.42 59.917244) (end 110.42 56.519899) (width 0.2) (layer "B.Cu") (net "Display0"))
 (segment (start 101.1125 47.212399) (end 101.1125 29.213478) (width 0.2) (layer "B.Cu") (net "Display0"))
 (segment (start 110.42 56.519899) (end 101.1125 47.212399) (width 0.2) (layer "B.Cu") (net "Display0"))
 (segment (start 108.2375 22.088478) (end 108.2375 21.011522) (width 0.2) (layer "B.Cu") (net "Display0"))
 (segment (start 108.2375 21.011522) (end 111.469022 17.78) (width 0.2) (layer "B.Cu") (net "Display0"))
 (segment (start 126.107944 67.775) (end 118.277756 67.775) (width 0.2) (layer "B.Cu") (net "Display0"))
 (segment (start 144.375 24.515) (end 144.375 52.902056) (width 0.2) (layer "B.Cu") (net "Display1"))
 (segment (start 118.11207 68.175) (end 98.9125 48.97543) (width 0.2) (layer "B.Cu") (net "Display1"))
 (segment (start 100.6375 23.35) (end 105.2375 23.35) (width 0.2) (layer "B.Cu") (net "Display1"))
 (segment (start 136.098629 58.35) (end 126.273629 68.175) (width 0.2) (layer "B.Cu") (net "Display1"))
 (segment (start 144.375 52.902056) (end 138.927056 58.35) (width 0.2) (layer "B.Cu") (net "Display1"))
 (segment (start 113.3475 15.24) (end 115.85 15.24) (width 0.2) (layer "B.Cu") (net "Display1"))
 (segment (start 141.45 21.59) (end 144.375 24.515) (width 0.2) (layer "B.Cu") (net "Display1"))
 (segment (start 98.9125 48.97543) (end 98.9125 25.075) (width 0.2) (layer "B.Cu") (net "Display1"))
 (segment (start 126.273629 68.175) (end 118.11207 68.175) (width 0.2) (layer "B.Cu") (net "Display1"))
 (segment (start 98.9125 25.075) (end 100.6375 23.35) (width 0.2) (layer "B.Cu") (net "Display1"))
 (segment (start 138.927056 58.35) (end 136.098629 58.35) (width 0.2) (layer "B.Cu") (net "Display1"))
 (segment (start 105.2375 23.35) (end 113.3475 15.24) (width 0.2) (layer "B.Cu") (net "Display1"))
 (segment (start 124.1425 35.56) (end 123.825 35.2425) (width 0.2) (layer "F.Cu") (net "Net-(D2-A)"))
 (segment (start 129.54 35.56) (end 124.1425 35.56) (width 0.2) (layer "F.Cu") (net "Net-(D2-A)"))
 (segment (start 146.3675 33.3375) (end 142.875 33.3375) (width 0.2) (layer "F.Cu") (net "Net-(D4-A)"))
 (segment (start 148.59 35.56) (end 146.3675 33.3375) (width 0.2) (layer "F.Cu") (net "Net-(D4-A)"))
 (segment (start 156.0625 67.775) (end 139.2125 67.775) (width 0.2) (layer "F.Cu") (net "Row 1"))
 (segment (start 139.2125 67.775) (end 138.1125 66.675) (width 0.2) (layer "F.Cu") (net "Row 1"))
 (segment (start 157.1625 66.675) (end 156.0625 67.775) (width 0.2) (layer "F.Cu") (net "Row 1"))
 (segment (start 119.0625 66.675) (end 111.89 59.5025) (width 0.2) (layer "F.Cu") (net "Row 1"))
 (segment (start 138.1125 66.675) (end 137.0125 67.775) (width 0.2) (layer "F.Cu") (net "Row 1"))
 (segment (start 120.1625 67.775) (end 119.0625 66.675) (width 0.2) (layer "F.Cu") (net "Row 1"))
 (segment (start 111.89 59.5025) (end 111.89 49.957244) (width 0.2) (layer "F.Cu") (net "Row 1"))
 (segment (start 111.89 49.957244) (end 100.0125 38.079744) (width 0.2) (layer "F.Cu") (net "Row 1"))
 (segment (start 100.0125 38.079744) (end 100.0125 36.195) (width 0.2) (layer "F.Cu") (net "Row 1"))
 (segment (start 137.0125 67.775) (end 120.1625 67.775) (width 0.2) (layer "F.Cu") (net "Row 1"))
 (segment (start 141.45 26.67) (end 141.45 40.720101) (width 0.2) (layer "B.Cu") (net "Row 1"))
 (segment (start 141.45 40.720101) (end 119.0625 63.107601) (width 0.2) (layer "B.Cu") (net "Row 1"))
 (segment (start 119.0625 63.107601) (end 119.0625 66.675) (width 0.2) (layer "B.Cu") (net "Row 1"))
 (segment (start 111.89 37.127056) (end 108.059556 40.9575) (width 0.2) (layer "F.Cu") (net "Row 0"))
 (segment (start 154.360101 31.62) (end 150.05 35.930101) (width 0.2) (layer "F.Cu") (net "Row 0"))
 (segment (start 146.159556 40.9575) (end 142.875 40.9575) (width 0.2) (layer "F.Cu") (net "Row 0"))
 (segment (start 131 37.067056) (end 125.204556 42.8625) (width 0.2) (layer "F.Cu") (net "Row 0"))
 (segment (start 136.469899 31.62) (end 135.310101 31.62) (width 0.2) (layer "F.Cu") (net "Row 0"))
 (segment (start 123.825 38.025101) (end 117.419899 31.62) (width 0.2) (layer "F.Cu") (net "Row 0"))
 (segment (start 150.05 37.067056) (end 146.159556 40.9575) (width 0.2) (layer "F.Cu") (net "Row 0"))
 (segment (start 142.875 40.9575) (end 142.875 38.025101) (width 0.2) (layer "F.Cu") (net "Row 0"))
 (segment (start 131 35.930101) (end 131 37.067056) (width 0.2) (layer "F.Cu") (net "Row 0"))
 (segment (start 108.059556 40.9575) (end 104.775 40.9575) (width 0.2) (layer "F.Cu") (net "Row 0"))
 (segment (start 125.204556 42.8625) (end 123.825 42.8625) (width 0.2) (layer "F.Cu") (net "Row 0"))
 (segment (start 166.6875 36.195) (end 162.1125 31.62) (width 0.2) (layer "F.Cu") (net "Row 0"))
 (segment (start 150.05 35.930101) (end 150.05 37.067056) (width 0.2) (layer "F.Cu") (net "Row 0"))
 (segment (start 111.89 35.7475) (end 111.89 37.127056) (width 0.2) (layer "F.Cu") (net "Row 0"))
 (segment (start 123.825 42.8625) (end 123.825 38.025101) (width 0.2) (layer "F.Cu") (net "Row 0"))
 (segment (start 162.1125 31.62) (end 154.360101 31.62) (width 0.2) (layer "F.Cu") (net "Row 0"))
 (segment (start 116.0175 31.62) (end 111.89 35.7475) (width 0.2) (layer "F.Cu") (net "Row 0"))
 (segment (start 117.419899 31.62) (end 116.0175 31.62) (width 0.2) (layer "F.Cu") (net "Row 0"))
 (segment (start 135.310101 31.62) (end 131 35.930101) (width 0.2) (layer "F.Cu") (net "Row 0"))
 (segment (start 142.875 38.025101) (end 136.469899 31.62) (width 0.2) (layer "F.Cu") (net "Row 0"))
 (segment (start 162.190686 7.425) (end 166.75 11.984315) (width 0.2) (layer "B.Cu") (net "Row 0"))
 (segment (start 93.7375 15.25) (end 101.5625 7.425) (width 0.2) (layer "B.Cu") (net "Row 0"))
 (segment (start 105.171814 22.85) (end 94.499022 22.85) (width 0.2) (layer "B.Cu") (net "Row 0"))
 (segment (start 117 18.256346) (end 117 14.763654) (width 0.2) (layer "B.Cu") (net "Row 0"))
 (segment (start 173.15 20.845837) (end 173.15 29.7325) (width 0.2) (layer "B.Cu") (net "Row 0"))
 (segment (start 166.75 11.984315) (end 166.75 14.445837) (width 0.2) (layer "B.Cu") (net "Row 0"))
 (segment (start 117 14.763654) (end 116.326346 14.09) (width 0.2) (layer "B.Cu") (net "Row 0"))
 (segment (start 113.931814 14.09) (end 105.171814 22.85) (width 0.2) (layer "B.Cu") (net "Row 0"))
 (segment (start 125.25 26.67) (end 117.064925 26.67) (width 0.2) (layer "B.Cu") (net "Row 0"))
 (segment (start 110.884707 18.93) (end 116.326346 18.93) (width 0.2) (layer "B.Cu") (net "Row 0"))
 (segment (start 110.104816 19.709891) (end 110.884707 18.93) (width 0.2) (layer "B.Cu") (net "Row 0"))
 (segment (start 173.15 29.7325) (end 166.6875 36.195) (width 0.2) (layer "B.Cu") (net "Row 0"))
 (segment (start 101.5625 7.425) (end 162.190686 7.425) (width 0.2) (layer "B.Cu") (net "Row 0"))
 (segment (start 117.064925 26.67) (end 110.104816 19.709891) (width 0.2) (layer "B.Cu") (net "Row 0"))
 (segment (start 94.499022 22.85) (end 93.7375 22.088478) (width 0.2) (layer "B.Cu") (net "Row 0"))
 (segment (start 116.326346 18.93) (end 117 18.256346) (width 0.2) (layer "B.Cu") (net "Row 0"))
 (segment (start 93.7375 22.088478) (end 93.7375 15.25) (width 0.2) (layer "B.Cu") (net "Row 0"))
 (segment (start 166.75 14.445837) (end 173.15 20.845837) (width 0.2) (layer "B.Cu") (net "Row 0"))
 (segment (start 116.326346 14.09) (end 113.931814 14.09) (width 0.2) (layer "B.Cu") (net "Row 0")))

